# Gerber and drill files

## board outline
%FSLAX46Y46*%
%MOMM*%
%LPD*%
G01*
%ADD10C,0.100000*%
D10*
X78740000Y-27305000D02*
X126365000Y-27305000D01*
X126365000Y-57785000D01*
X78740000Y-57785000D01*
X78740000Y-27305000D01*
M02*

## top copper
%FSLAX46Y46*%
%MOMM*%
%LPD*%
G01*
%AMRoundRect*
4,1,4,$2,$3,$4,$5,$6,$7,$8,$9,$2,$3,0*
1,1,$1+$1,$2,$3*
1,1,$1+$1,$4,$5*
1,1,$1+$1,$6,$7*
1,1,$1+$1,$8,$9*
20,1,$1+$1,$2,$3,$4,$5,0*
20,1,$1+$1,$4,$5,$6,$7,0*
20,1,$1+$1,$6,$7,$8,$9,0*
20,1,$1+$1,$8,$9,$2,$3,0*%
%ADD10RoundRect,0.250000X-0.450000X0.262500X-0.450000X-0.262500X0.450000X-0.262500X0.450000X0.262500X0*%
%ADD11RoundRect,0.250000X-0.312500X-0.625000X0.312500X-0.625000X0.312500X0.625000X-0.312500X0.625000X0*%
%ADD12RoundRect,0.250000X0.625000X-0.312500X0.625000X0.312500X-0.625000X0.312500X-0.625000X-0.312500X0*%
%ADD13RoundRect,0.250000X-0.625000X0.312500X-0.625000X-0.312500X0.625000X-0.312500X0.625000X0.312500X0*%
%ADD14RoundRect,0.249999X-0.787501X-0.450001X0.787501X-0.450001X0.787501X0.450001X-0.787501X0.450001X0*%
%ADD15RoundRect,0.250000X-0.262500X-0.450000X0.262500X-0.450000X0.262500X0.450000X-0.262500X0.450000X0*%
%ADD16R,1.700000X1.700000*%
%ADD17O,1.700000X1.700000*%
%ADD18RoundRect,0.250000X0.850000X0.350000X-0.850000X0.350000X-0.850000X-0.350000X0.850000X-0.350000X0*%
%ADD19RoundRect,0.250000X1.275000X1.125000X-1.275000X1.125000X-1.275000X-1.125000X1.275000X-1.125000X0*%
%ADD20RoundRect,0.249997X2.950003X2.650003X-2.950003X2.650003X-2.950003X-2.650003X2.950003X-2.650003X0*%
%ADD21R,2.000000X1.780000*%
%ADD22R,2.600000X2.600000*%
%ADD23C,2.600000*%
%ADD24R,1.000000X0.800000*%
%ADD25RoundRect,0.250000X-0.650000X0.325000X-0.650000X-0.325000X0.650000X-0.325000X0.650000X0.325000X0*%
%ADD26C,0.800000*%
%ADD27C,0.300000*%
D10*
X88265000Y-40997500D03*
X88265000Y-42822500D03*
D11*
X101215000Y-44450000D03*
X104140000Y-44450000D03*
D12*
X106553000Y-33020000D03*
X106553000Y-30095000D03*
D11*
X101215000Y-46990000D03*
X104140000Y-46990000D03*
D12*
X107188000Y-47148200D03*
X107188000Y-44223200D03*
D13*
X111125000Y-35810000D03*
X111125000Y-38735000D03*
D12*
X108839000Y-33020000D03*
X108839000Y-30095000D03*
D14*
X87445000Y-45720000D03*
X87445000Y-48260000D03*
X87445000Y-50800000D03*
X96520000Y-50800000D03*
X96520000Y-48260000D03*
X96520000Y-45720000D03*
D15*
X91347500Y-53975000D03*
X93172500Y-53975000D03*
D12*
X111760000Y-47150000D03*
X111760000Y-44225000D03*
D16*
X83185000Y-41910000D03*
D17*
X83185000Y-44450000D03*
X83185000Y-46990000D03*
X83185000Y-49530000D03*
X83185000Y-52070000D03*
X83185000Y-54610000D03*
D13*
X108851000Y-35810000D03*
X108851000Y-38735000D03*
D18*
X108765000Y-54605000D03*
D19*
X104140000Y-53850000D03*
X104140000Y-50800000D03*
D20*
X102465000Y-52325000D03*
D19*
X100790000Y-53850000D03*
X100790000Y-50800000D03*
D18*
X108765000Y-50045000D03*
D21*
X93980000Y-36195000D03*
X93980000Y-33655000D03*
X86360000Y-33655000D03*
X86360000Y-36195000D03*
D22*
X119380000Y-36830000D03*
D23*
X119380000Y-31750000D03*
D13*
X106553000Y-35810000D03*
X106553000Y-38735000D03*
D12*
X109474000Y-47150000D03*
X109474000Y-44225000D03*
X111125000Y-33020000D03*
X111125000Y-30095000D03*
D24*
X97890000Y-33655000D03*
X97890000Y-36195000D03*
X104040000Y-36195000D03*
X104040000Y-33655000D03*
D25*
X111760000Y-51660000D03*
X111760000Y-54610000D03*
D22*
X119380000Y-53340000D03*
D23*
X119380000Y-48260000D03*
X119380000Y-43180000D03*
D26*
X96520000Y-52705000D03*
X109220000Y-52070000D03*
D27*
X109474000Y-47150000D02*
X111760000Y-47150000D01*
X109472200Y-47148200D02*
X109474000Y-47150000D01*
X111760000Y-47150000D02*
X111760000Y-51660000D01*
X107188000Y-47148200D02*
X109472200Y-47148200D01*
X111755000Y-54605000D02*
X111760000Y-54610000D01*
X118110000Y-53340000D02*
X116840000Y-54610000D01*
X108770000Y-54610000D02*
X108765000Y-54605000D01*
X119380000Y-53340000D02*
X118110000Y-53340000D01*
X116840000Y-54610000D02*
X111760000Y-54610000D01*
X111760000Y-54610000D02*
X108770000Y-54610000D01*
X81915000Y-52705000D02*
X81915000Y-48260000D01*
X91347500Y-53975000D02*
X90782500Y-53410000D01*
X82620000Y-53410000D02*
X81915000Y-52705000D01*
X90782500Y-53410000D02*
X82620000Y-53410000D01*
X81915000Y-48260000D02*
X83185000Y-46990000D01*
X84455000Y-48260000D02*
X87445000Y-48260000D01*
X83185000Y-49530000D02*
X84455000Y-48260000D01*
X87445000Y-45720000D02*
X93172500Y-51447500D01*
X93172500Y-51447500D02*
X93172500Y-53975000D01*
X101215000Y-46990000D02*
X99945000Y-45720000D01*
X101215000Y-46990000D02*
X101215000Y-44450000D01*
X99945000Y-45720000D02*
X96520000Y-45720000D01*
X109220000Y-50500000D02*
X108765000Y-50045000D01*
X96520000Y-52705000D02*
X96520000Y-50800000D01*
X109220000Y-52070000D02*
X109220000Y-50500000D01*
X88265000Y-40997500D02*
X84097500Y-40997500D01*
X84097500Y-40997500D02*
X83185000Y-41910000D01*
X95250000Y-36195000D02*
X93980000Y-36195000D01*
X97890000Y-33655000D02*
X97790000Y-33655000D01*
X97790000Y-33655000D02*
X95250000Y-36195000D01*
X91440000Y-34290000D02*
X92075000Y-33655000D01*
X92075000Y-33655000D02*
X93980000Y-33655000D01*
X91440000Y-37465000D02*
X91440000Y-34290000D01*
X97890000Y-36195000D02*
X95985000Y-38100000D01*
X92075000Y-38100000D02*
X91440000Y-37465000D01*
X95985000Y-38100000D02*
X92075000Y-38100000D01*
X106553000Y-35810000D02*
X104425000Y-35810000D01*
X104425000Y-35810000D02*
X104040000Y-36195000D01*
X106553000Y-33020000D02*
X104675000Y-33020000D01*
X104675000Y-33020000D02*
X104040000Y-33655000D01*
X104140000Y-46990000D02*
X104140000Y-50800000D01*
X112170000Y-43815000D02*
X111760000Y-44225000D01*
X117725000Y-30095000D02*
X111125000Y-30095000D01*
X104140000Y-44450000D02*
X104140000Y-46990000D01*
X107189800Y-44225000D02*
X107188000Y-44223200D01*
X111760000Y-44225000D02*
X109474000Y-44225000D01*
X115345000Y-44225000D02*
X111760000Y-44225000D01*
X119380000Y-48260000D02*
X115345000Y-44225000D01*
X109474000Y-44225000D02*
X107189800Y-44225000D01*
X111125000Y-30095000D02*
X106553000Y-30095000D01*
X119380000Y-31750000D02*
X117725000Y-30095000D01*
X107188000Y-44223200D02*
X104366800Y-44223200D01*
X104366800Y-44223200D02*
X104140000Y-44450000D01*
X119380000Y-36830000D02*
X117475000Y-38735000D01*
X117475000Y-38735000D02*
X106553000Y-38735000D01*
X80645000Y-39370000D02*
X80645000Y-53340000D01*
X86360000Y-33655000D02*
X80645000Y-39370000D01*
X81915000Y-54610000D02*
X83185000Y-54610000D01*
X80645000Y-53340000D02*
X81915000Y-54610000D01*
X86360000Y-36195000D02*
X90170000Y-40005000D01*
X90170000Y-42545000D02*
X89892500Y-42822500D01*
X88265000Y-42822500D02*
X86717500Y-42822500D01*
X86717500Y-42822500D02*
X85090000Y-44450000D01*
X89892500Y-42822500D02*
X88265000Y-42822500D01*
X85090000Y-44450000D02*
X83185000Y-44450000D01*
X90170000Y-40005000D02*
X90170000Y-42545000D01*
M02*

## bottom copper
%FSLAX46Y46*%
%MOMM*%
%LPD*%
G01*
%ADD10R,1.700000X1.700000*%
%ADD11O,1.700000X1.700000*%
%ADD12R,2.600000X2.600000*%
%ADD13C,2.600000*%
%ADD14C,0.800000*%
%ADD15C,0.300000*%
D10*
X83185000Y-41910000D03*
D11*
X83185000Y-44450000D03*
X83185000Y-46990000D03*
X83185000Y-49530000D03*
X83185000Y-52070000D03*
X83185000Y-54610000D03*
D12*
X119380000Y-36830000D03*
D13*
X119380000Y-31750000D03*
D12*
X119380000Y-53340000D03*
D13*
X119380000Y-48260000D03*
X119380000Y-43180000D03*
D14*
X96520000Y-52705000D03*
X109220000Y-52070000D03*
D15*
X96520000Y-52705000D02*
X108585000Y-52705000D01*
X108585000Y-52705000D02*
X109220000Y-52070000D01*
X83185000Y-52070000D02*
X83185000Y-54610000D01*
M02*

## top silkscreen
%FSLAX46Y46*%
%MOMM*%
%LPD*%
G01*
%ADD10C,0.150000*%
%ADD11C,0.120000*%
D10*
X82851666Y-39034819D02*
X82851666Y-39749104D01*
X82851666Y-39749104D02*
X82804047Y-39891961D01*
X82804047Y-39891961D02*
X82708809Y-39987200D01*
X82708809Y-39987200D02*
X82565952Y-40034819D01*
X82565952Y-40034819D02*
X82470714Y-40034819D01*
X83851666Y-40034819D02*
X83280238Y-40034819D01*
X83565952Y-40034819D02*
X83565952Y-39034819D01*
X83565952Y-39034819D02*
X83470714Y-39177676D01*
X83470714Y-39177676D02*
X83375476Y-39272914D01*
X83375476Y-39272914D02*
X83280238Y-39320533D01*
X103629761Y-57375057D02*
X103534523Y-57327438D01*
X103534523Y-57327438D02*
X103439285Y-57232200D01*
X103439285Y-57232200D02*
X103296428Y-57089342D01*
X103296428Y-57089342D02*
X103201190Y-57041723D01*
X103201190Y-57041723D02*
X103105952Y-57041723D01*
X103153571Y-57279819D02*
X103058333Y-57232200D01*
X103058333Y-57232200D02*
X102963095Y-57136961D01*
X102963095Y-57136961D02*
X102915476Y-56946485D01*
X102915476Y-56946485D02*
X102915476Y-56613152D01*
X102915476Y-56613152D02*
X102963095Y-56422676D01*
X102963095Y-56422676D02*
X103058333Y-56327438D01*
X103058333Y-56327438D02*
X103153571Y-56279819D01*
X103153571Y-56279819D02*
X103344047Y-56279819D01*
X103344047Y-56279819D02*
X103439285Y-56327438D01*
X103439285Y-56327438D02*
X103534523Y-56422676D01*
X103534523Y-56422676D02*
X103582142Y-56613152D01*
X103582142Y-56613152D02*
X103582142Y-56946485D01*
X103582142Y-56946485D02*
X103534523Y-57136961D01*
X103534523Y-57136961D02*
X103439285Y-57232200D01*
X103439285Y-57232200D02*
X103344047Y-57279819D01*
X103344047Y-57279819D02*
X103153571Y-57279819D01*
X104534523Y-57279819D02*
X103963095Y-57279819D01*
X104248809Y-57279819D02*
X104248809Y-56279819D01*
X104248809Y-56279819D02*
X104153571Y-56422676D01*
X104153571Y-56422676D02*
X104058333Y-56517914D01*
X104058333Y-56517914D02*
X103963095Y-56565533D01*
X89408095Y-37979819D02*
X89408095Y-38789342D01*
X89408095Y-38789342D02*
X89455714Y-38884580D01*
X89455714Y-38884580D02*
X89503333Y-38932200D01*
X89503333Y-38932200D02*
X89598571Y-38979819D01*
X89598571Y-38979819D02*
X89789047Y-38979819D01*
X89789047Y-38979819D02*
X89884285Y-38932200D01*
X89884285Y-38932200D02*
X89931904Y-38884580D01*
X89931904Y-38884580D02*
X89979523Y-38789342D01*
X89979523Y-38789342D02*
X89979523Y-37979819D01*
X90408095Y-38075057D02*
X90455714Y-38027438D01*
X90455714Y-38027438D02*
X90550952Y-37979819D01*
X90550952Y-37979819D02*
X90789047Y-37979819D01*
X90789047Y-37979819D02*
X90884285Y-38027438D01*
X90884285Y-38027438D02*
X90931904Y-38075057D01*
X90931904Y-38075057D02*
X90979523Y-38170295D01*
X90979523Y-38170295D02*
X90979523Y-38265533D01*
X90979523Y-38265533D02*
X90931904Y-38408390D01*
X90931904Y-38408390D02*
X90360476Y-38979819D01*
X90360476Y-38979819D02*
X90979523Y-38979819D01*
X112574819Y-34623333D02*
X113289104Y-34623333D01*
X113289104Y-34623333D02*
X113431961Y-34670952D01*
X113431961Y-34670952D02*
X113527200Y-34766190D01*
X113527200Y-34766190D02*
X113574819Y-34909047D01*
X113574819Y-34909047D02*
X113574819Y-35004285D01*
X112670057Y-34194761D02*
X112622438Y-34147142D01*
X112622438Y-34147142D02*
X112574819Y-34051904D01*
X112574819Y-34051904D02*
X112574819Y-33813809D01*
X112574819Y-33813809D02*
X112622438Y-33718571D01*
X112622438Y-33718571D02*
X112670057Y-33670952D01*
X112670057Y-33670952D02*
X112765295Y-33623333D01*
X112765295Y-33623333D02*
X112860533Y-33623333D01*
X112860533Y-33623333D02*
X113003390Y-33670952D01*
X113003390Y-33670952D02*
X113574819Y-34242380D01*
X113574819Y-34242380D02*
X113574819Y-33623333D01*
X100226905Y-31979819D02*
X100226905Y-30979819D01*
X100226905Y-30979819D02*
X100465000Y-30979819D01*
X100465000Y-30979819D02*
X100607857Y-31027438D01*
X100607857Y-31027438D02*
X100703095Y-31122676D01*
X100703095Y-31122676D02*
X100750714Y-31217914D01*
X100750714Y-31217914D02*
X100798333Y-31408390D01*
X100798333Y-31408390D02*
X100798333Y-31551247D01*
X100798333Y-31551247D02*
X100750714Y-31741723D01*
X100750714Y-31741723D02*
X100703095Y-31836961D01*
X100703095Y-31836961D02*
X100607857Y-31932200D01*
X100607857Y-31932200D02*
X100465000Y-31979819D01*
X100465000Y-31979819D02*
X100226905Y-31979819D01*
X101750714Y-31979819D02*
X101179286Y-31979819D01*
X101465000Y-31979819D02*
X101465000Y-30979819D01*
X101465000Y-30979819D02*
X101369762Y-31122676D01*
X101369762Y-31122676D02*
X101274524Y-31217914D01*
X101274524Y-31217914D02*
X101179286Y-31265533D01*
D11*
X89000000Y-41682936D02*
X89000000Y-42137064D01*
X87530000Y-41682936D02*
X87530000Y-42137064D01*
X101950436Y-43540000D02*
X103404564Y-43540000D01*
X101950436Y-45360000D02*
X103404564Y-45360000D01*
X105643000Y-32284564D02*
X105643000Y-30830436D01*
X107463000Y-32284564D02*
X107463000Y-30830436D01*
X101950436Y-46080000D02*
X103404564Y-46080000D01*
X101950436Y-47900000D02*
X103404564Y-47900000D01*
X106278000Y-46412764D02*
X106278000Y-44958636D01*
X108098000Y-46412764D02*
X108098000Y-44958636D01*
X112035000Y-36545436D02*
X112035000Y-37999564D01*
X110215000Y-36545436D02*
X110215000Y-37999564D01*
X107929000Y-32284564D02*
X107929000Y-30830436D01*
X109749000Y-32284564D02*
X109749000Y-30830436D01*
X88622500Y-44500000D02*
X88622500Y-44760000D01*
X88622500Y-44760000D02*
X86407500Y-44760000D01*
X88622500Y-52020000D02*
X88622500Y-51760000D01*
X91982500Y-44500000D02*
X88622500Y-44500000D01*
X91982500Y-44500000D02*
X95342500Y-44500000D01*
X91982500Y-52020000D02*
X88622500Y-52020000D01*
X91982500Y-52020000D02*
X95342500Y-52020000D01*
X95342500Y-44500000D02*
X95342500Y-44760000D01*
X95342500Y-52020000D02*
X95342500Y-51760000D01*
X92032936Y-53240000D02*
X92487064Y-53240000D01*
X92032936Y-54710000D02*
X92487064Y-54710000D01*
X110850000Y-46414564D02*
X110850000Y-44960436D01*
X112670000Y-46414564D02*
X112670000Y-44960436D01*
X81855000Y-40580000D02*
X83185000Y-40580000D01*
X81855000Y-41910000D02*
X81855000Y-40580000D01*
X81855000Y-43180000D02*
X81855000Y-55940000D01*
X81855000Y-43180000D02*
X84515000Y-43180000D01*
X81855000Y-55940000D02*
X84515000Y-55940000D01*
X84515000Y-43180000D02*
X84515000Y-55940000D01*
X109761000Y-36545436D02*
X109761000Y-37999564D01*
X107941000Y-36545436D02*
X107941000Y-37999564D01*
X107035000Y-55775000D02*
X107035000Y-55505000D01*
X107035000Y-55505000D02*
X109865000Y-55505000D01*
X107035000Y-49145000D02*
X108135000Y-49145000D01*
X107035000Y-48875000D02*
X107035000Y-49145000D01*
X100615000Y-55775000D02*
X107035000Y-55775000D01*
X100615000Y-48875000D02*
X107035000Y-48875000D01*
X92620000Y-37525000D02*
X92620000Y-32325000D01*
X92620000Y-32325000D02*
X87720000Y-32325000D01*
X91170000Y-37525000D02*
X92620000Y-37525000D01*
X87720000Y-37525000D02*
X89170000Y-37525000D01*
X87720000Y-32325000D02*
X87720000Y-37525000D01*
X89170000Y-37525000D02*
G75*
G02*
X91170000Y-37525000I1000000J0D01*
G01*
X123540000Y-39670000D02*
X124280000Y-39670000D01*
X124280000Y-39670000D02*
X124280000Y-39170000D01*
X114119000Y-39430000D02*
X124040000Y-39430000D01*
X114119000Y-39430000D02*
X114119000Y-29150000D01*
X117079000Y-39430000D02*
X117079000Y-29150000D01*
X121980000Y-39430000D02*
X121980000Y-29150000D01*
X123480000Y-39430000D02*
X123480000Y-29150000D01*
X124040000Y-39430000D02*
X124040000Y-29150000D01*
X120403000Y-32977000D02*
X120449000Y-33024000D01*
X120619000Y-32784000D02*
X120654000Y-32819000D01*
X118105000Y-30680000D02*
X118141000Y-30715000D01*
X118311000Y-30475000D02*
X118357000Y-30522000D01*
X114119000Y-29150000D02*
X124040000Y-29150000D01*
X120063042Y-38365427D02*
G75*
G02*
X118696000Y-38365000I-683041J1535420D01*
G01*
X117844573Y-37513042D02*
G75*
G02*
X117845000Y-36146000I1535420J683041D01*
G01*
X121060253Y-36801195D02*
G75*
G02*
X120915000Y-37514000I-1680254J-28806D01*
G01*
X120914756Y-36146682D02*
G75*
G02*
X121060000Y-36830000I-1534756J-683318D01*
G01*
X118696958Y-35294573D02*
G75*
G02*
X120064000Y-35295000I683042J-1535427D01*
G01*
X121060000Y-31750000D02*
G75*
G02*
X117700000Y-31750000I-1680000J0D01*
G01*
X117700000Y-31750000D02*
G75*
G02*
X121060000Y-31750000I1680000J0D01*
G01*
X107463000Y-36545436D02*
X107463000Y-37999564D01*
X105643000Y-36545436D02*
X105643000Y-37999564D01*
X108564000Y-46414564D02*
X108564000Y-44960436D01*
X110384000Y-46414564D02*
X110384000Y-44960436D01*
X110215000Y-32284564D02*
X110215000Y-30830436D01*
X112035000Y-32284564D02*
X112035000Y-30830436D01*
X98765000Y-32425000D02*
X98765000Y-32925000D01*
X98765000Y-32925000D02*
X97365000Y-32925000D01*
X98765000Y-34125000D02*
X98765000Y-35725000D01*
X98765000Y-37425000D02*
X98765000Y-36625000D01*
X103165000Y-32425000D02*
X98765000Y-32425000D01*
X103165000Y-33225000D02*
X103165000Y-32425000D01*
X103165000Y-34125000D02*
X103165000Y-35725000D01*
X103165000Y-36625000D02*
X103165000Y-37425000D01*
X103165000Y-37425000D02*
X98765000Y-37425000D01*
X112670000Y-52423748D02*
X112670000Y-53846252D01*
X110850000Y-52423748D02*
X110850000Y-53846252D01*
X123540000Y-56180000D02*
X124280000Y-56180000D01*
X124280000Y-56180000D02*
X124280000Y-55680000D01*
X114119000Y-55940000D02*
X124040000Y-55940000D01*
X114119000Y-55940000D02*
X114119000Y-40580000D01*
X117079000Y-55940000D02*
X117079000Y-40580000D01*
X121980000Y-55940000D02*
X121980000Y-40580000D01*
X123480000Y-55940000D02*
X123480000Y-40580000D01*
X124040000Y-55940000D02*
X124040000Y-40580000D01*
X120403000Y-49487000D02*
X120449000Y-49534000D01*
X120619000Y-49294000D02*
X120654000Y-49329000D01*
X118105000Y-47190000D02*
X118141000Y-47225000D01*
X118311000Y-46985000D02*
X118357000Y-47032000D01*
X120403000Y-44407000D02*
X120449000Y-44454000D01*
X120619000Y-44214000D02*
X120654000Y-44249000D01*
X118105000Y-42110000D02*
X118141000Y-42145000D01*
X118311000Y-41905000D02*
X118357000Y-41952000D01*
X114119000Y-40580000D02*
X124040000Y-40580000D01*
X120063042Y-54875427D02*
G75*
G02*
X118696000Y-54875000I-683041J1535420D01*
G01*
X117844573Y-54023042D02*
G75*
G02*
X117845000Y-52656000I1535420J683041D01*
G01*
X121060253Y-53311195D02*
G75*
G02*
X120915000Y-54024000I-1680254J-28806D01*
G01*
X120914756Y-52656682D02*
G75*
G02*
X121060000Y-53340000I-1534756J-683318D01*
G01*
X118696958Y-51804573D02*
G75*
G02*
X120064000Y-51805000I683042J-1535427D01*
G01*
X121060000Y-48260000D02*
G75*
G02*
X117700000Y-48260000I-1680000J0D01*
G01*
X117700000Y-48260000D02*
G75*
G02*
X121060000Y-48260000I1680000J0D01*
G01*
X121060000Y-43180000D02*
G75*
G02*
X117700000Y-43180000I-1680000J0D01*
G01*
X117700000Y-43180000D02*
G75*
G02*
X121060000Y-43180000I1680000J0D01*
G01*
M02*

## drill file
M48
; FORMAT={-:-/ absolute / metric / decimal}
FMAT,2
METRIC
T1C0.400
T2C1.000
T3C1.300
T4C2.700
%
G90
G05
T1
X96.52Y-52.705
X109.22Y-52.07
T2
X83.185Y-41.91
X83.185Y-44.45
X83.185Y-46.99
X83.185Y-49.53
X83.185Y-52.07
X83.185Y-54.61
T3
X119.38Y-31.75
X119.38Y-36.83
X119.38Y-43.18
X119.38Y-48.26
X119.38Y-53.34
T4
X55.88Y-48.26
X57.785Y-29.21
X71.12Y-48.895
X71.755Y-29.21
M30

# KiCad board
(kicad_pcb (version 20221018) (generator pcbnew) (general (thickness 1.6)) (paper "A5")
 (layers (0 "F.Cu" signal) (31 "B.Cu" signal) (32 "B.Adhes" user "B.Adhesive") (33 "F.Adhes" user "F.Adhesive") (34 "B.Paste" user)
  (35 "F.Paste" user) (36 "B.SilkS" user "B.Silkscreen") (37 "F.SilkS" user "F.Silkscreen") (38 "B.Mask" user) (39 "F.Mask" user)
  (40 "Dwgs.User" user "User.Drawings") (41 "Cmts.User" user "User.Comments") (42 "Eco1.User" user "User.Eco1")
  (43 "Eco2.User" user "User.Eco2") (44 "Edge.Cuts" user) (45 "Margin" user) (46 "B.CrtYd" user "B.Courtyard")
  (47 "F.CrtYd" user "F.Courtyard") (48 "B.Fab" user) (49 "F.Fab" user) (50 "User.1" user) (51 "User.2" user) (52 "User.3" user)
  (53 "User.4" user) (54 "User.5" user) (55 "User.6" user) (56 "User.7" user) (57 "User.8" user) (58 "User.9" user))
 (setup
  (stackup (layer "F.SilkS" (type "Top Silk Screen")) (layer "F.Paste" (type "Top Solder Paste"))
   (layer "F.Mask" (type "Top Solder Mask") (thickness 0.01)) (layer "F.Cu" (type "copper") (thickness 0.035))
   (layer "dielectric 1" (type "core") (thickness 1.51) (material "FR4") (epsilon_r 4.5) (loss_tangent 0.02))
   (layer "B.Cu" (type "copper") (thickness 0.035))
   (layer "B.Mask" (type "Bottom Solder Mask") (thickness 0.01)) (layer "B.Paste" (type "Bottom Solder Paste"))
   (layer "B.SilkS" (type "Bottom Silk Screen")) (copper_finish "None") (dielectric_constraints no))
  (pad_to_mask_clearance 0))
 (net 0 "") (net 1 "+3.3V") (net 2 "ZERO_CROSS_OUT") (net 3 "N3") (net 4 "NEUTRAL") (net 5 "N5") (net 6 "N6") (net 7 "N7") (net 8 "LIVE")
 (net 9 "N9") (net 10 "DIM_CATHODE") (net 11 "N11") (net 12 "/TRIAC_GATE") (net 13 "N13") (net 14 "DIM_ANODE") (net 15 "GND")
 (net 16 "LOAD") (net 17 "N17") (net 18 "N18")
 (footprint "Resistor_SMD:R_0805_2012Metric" (layer "F.Cu") (at 88.265 41.91 -90)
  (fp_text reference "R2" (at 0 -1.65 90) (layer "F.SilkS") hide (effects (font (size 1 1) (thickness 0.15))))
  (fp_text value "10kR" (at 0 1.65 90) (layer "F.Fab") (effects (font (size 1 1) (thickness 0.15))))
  (fp_line (start -0.227064 -0.735) (end 0.227064 -0.735) (stroke (width 0.12) (type solid)) (layer "F.SilkS"))
  (fp_line (start -0.227064 0.735) (end 0.227064 0.735) (stroke (width 0.12) (type solid)) (layer "F.SilkS"))
  (pad "1" smd roundrect (at -0.9125 0 270) (size 1.025 1.4) (layers "F.Cu" "F.Paste" "F.Mask") (roundrect_rratio 0.243902) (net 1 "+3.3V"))
  (pad "2" smd roundrect (at 0.9125 0 270) (size 1.025 1.4) (layers "F.Cu" "F.Paste" "F.Mask") (roundrect_rratio 0.243902)
   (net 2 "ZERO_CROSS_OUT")))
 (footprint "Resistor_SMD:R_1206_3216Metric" (layer "F.Cu") (at 102.6775 44.45)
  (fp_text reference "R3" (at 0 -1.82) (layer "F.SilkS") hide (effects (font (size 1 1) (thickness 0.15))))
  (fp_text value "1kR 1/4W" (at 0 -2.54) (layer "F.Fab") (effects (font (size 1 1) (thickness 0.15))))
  (fp_line (start -0.727064 -0.91) (end 0.727064 -0.91) (stroke (width 0.12) (type solid)) (layer "F.SilkS"))
  (fp_line (start -0.727064 0.91) (end 0.727064 0.91) (stroke (width 0.12) (type solid)) (layer "F.SilkS"))
  (pad "1" smd roundrect (at -1.4625 0) (size 1.125 1.75) (layers "F.Cu" "F.Paste" "F.Mask") (roundrect_rratio 0.2222222222) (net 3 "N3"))
  (pad "2" smd roundrect (at 1.4625 0) (size 1.125 1.75) (layers "F.Cu" "F.Paste" "F.Mask") (roundrect_rratio 0.2222222222)
   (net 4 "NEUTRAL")))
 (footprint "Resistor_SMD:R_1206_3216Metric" (layer "F.Cu") (at 106.553 31.5575 90)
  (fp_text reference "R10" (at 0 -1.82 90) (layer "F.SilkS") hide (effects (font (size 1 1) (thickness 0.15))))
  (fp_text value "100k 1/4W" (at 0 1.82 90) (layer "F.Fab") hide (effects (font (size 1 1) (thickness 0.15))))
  (fp_line (start -0.727064 -0.91) (end 0.727064 -0.91) (stroke (width 0.12) (type solid)) (layer "F.SilkS"))
  (fp_line (start -0.727064 0.91) (end 0.727064 0.91) (stroke (width 0.12) (type solid)) (layer "F.SilkS"))
  (pad "1" smd roundrect (at -1.4625 0 90) (size 1.125 1.75) (layers "F.Cu" "F.Paste" "F.Mask") (roundrect_rratio 0.222222) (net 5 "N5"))
  (pad "2" smd roundrect (at 1.4625 0 90) (size 1.125 1.75) (layers "F.Cu" "F.Paste" "F.Mask") (roundrect_rratio 0.222222) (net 4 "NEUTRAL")))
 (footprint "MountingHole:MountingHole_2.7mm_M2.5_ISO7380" (layer "F.Cu") (at 71.755 29.21)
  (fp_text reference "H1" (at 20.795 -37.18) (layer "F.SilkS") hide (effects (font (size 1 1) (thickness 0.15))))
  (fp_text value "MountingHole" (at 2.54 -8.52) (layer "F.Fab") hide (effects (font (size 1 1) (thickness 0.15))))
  (pad "" np_thru_hole circle (at 0 0) (size 2.7 2.7) (drill 2.7) (layers "*.Cu" "*.Mask")))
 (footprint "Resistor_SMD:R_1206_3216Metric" (layer "F.Cu") (at 102.6775 46.99)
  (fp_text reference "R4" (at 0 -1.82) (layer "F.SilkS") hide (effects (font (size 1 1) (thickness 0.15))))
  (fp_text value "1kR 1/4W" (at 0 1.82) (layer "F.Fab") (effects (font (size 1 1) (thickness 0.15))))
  (fp_line (start -0.727064 -0.91) (end 0.727064 -0.91) (stroke (width 0.12) (type solid)) (layer "F.SilkS"))
  (fp_line (start -0.727064 0.91) (end 0.727064 0.91) (stroke (width 0.12) (type solid)) (layer "F.SilkS"))
  (pad "1" smd roundrect (at -1.4625 0) (size 1.125 1.75) (layers "F.Cu" "F.Paste" "F.Mask") (roundrect_rratio 0.2222222222) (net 3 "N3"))
  (pad "2" smd roundrect (at 1.4625 0) (size 1.125 1.75) (layers "F.Cu" "F.Paste" "F.Mask") (roundrect_rratio 0.2222222222)
   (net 4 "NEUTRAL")))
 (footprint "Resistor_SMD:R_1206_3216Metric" (layer "F.Cu") (at 107.188 45.6857 90)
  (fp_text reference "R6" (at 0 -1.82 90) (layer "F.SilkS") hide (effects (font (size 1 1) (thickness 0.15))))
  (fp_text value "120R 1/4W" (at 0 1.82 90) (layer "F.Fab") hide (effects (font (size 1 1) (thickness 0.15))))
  (fp_line (start -0.727064 -0.91) (end 0.727064 -0.91) (stroke (width 0.12) (type solid)) (layer "F.SilkS"))
  (fp_line (start -0.727064 0.91) (end 0.727064 0.91) (stroke (width 0.12) (type solid)) (layer "F.SilkS"))
  (pad "1" smd roundrect (at -1.4625 0 90) (size 1.125 1.75) (layers "F.Cu" "F.Paste" "F.Mask") (roundrect_rratio 0.222222) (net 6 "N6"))
  (pad "2" smd roundrect (at 1.4625 0 90) (size 1.125 1.75) (layers "F.Cu" "F.Paste" "F.Mask") (roundrect_rratio 0.222222) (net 4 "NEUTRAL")))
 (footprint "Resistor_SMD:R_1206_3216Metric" (layer "F.Cu") (at 111.125 37.2725 -90)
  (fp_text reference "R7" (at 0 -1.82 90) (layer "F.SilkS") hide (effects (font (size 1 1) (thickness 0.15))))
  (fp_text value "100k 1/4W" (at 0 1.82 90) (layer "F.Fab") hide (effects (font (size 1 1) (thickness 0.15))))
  (fp_line (start -0.727064 -0.91) (end 0.727064 -0.91) (stroke (width 0.12) (type solid)) (layer "F.SilkS"))
  (fp_line (start -0.727064 0.91) (end 0.727064 0.91) (stroke (width 0.12) (type solid)) (layer "F.SilkS"))
  (pad "1" smd roundrect (at -1.4625 0 270) (size 1.125 1.75) (layers "F.Cu" "F.Paste" "F.Mask") (roundrect_rratio 0.222222) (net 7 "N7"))
  (pad "2" smd roundrect (at 1.4625 0 270) (size 1.125 1.75) (layers "F.Cu" "F.Paste" "F.Mask") (roundrect_rratio 0.222222) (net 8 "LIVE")))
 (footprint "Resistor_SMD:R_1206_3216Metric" (layer "F.Cu") (at 108.839 31.5575 90)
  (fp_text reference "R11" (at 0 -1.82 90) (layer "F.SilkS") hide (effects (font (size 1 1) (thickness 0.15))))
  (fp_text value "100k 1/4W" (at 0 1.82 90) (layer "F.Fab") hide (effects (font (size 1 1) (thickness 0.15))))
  (fp_line (start -0.727064 -0.91) (end 0.727064 -0.91) (stroke (width 0.12) (type solid)) (layer "F.SilkS"))
  (fp_line (start -0.727064 0.91) (end 0.727064 0.91) (stroke (width 0.12) (type solid)) (layer "F.SilkS"))
  (pad "1" smd roundrect (at -1.4625 0 90) (size 1.125 1.75) (layers "F.Cu" "F.Paste" "F.Mask") (roundrect_rratio 0.222222) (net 5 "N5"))
  (pad "2" smd roundrect (at 1.4625 0 90) (size 1.125 1.75) (layers "F.Cu" "F.Paste" "F.Mask") (roundrect_rratio 0.222222) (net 4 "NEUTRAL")))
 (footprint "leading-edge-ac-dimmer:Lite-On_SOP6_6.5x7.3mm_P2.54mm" (layer "F.Cu") (at 91.9825 48.26)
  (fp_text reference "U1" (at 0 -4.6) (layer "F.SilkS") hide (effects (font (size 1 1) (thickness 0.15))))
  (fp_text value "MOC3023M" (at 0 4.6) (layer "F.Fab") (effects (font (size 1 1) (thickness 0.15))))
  (fp_line (start -3.36 -3.76) (end -3.36 -3.5) (stroke (width 0.12) (type solid)) (layer "F.SilkS"))
  (fp_line (start -3.36 -3.5) (end -5.575 -3.5) (stroke (width 0.12) (type solid)) (layer "F.SilkS"))
  (fp_line (start -3.36 3.76) (end -3.36 3.5) (stroke (width 0.12) (type solid)) (layer "F.SilkS"))
  (fp_line (start 0 -3.76) (end -3.36 -3.76) (stroke (width 0.12) (type solid)) (layer "F.SilkS"))
  (fp_line (start 0 -3.76) (end 3.36 -3.76) (stroke (width 0.12) (type solid)) (layer "F.SilkS"))
  (fp_line (start 0 3.76) (end -3.36 3.76) (stroke (width 0.12) (type solid)) (layer "F.SilkS"))
  (fp_line (start 0 3.76) (end 3.36 3.76) (stroke (width 0.12) (type solid)) (layer "F.SilkS"))
  (fp_line (start 3.36 -3.76) (end 3.36 -3.5) (stroke (width 0.12) (type solid)) (layer "F.SilkS"))
  (fp_line (start 3.36 3.76) (end 3.36 3.5) (stroke (width 0.12) (type solid)) (layer "F.SilkS"))
  (pad "1" smd roundrect (at -4.5375 -2.54) (size 2.075 1.4) (layers "F.Cu" "F.Paste" "F.Mask") (roundrect_rratio 0.178571) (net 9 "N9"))
  (pad "2" smd roundrect (at -4.5375 0) (size 2.075 1.4) (layers "F.Cu" "F.Paste" "F.Mask") (roundrect_rratio 0.178571)
   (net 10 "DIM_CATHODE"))
  (pad "3" smd roundrect (at -4.5375 2.54) (size 2.075 1.4) (layers "F.Cu" "F.Paste" "F.Mask") (roundrect_rratio 0.178571) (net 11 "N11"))
  (pad "4" smd roundrect (at 4.5375 2.54) (size 2.075 1.4) (layers "F.Cu" "F.Paste" "F.Mask") (roundrect_rratio 0.178571)
   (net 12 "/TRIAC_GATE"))
  (pad "5" smd roundrect (at 4.5375 0) (size 2.075 1.4) (layers "F.Cu" "F.Paste" "F.Mask") (roundrect_rratio 0.178571) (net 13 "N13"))
  (pad "6" smd roundrect (at 4.5375 -2.54) (size 2.075 1.4) (layers "F.Cu" "F.Paste" "F.Mask") (roundrect_rratio 0.178571) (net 3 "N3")))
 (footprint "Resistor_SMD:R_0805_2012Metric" (layer "F.Cu") (at 92.26 53.975)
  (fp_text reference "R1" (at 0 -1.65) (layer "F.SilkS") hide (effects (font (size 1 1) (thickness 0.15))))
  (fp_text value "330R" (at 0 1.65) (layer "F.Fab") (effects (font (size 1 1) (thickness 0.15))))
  (fp_line (start -0.227064 -0.735) (end 0.227064 -0.735) (stroke (width 0.12) (type solid)) (layer "F.SilkS"))
  (fp_line (start -0.227064 0.735) (end 0.227064 0.735) (stroke (width 0.12) (type solid)) (layer "F.SilkS"))
  (pad "1" smd roundrect (at -0.9125 0) (size 1.025 1.4) (layers "F.Cu" "F.Paste" "F.Mask") (roundrect_rratio 0.243902) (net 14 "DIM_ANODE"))
  (pad "2" smd roundrect (at 0.9125 0) (size 1.025 1.4) (layers "F.Cu" "F.Paste" "F.Mask") (roundrect_rratio 0.243902) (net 9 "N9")))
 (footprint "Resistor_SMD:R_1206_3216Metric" (layer "F.Cu") (at 111.76 45.6875 90)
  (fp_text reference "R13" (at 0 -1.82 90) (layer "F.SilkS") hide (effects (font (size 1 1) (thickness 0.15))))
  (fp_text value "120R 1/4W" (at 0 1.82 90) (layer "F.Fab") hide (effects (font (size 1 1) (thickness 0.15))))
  (fp_line (start -0.727064 -0.91) (end 0.727064 -0.91) (stroke (width 0.12) (type solid)) (layer "F.SilkS"))
  (fp_line (start -0.727064 0.91) (end 0.727064 0.91) (stroke (width 0.12) (type solid)) (layer "F.SilkS"))
  (pad "1" smd roundrect (at -1.4625 0 90) (size 1.125 1.75) (layers "F.Cu" "F.Paste" "F.Mask") (roundrect_rratio 0.222222) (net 6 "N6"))
  (pad "2" smd roundrect (at 1.4625 0 90) (size 1.125 1.75) (layers "F.Cu" "F.Paste" "F.Mask") (roundrect_rratio 0.222222) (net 4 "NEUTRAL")))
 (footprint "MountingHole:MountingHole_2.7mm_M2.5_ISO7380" (layer "F.Cu") (at 55.88 48.26)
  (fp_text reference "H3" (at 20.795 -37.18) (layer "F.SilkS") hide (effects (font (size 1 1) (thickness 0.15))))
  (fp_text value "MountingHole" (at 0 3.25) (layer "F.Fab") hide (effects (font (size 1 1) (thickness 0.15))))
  (pad "" np_thru_hole circle (at 0 0) (size 2.7 2.7) (drill 2.7) (layers "*.Cu" "*.Mask")))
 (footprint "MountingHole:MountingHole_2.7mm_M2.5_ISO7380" (layer "F.Cu") (at 57.785 29.21)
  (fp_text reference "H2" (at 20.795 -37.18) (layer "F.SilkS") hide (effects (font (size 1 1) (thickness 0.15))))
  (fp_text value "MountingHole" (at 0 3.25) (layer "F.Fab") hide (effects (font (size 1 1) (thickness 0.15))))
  (pad "" np_thru_hole circle (at 0 0) (size 2.7 2.7) (drill 2.7) (layers "*.Cu" "*.Mask")))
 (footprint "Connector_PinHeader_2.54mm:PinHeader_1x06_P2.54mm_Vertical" (layer "F.Cu") (at 83.185 41.91)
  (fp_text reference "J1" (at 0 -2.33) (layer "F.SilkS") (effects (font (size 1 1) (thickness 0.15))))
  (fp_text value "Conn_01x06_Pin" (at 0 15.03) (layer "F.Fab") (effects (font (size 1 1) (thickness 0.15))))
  (fp_line (start -1.33 -1.33) (end 0 -1.33) (stroke (width 0.12) (type solid)) (layer "F.SilkS"))
  (fp_line (start -1.33 0) (end -1.33 -1.33) (stroke (width 0.12) (type solid)) (layer "F.SilkS"))
  (fp_line (start -1.33 1.27) (end -1.33 14.03) (stroke (width 0.12) (type solid)) (layer "F.SilkS"))
  (fp_line (start -1.33 1.27) (end 1.33 1.27) (stroke (width 0.12) (type solid)) (layer "F.SilkS"))
  (fp_line (start -1.33 14.03) (end 1.33 14.03) (stroke (width 0.12) (type solid)) (layer "F.SilkS"))
  (fp_line (start 1.33 1.27) (end 1.33 14.03) (stroke (width 0.12) (type solid)) (layer "F.SilkS"))
  (pad "1" thru_hole rect (at 0 0) (size 1.7 1.7) (drill 1) (layers "*.Cu" "*.Mask") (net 1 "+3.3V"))
  (pad "2" thru_hole oval (at 0 2.54) (size 1.7 1.7) (drill 1) (layers "*.Cu" "*.Mask") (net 2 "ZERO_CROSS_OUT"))
  (pad "3" thru_hole oval (at 0 5.08) (size 1.7 1.7) (drill 1) (layers "*.Cu" "*.Mask") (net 14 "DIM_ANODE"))
  (pad "4" thru_hole oval (at 0 7.62) (size 1.7 1.7) (drill 1) (layers "*.Cu" "*.Mask") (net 10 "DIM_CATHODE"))
  (pad "5" thru_hole oval (at 0 10.16) (size 1.7 1.7) (drill 1) (layers "*.Cu" "*.Mask") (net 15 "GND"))
  (pad "6" thru_hole oval (at 0 12.7) (size 1.7 1.7) (drill 1) (layers "*.Cu" "*.Mask") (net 15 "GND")))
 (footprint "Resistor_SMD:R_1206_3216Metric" (layer "F.Cu") (at 108.851 37.2725 -90)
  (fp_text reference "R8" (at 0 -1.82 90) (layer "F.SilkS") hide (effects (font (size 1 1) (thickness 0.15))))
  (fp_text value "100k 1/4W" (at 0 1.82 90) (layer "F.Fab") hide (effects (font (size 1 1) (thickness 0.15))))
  (fp_line (start -0.727064 -0.91) (end 0.727064 -0.91) (stroke (width 0.12) (type solid)) (layer "F.SilkS"))
  (fp_line (start -0.727064 0.91) (end 0.727064 0.91) (stroke (width 0.12) (type solid)) (layer "F.SilkS"))
  (pad "1" smd roundrect (at -1.4625 0 270) (size 1.125 1.75) (layers "F.Cu" "F.Paste" "F.Mask") (roundrect_rratio 0.222222) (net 7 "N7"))
  (pad "2" smd roundrect (at 1.4625 0 270) (size 1.125 1.75) (layers "F.Cu" "F.Paste" "F.Mask") (roundrect_rratio 0.222222) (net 8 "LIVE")))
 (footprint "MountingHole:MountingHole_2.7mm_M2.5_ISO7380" (layer "F.Cu") (at 71.12 48.895)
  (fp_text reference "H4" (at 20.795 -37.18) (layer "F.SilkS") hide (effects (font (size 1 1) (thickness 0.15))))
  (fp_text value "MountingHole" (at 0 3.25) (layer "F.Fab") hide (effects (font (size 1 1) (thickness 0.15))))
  (pad "" np_thru_hole circle (at 0 0) (size 2.7 2.7) (drill 2.7) (layers "*.Cu" "*.Mask")))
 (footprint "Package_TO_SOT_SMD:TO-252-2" (layer "F.Cu") (at 103.725 52.325 180)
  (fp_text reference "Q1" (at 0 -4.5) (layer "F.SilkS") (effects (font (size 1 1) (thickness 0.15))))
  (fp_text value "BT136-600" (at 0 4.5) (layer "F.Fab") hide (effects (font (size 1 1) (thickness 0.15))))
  (fp_line (start -3.31 -3.45) (end -3.31 -3.18) (stroke (width 0.12) (type solid)) (layer "F.SilkS"))
  (fp_line (start -3.31 -3.18) (end -6.14 -3.18) (stroke (width 0.12) (type solid)) (layer "F.SilkS"))
  (fp_line (start -3.31 3.18) (end -4.41 3.18) (stroke (width 0.12) (type solid)) (layer "F.SilkS"))
  (fp_line (start -3.31 3.45) (end -3.31 3.18) (stroke (width 0.12) (type solid)) (layer "F.SilkS"))
  (fp_line (start 3.11 -3.45) (end -3.31 -3.45) (stroke (width 0.12) (type solid)) (layer "F.SilkS"))
  (fp_line (start 3.11 3.45) (end -3.31 3.45) (stroke (width 0.12) (type solid)) (layer "F.SilkS"))
  (pad "1" smd roundrect (at -5.04 -2.28 180) (size 2.2 1.2) (layers "F.Cu" "F.Paste" "F.Mask") (roundrect_rratio 0.208333) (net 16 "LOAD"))
  (pad "2" smd roundrect (at -0.415 -1.525 180) (size 3.05 2.75) (layers "F.Cu" "F.Paste") (roundrect_rratio 0.090909) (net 4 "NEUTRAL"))
  (pad "2" smd roundrect (at -0.415 1.525 180) (size 3.05 2.75) (layers "F.Cu" "F.Paste") (roundrect_rratio 0.090909) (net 4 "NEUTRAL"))
  (pad "2" smd roundrect (at 1.26 0 180) (size 6.4 5.8) (layers "F.Cu" "F.Mask") (roundrect_rratio 0.043103) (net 4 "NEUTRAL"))
  (pad "2" smd roundrect (at 2.935 -1.525 180) (size 3.05 2.75) (layers "F.Cu" "F.Paste") (roundrect_rratio 0.090909) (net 4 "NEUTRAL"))
  (pad "2" smd roundrect (at 2.935 1.525 180) (size 3.05 2.75) (layers "F.Cu" "F.Paste") (roundrect_rratio 0.090909) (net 4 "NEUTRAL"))
  (pad "3" smd roundrect (at -5.04 2.28 180) (size 2.2 1.2) (layers "F.Cu" "F.Paste" "F.Mask") (roundrect_rratio 0.208333)
   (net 12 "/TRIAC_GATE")))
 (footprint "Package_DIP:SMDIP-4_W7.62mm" (layer "F.Cu") (at 90.17 34.925 180)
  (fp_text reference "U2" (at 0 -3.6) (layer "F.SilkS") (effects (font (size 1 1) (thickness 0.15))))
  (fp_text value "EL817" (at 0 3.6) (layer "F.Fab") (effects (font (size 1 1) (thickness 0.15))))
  (fp_line (start -2.45 -2.6) (end -2.45 2.6) (stroke (width 0.12) (type solid)) (layer "F.SilkS"))
  (fp_line (start -2.45 2.6) (end 2.45 2.6) (stroke (width 0.12) (type solid)) (layer "F.SilkS"))
  (fp_line (start -1 -2.6) (end -2.45 -2.6) (stroke (width 0.12) (type solid)) (layer "F.SilkS"))
  (fp_line (start 2.45 -2.6) (end 1 -2.6) (stroke (width 0.12) (type solid)) (layer "F.SilkS"))
  (fp_line (start 2.45 2.6) (end 2.45 -2.6) (stroke (width 0.12) (type solid)) (layer "F.SilkS"))
  (fp_arc (start 1 -2.6) (mid 0 -1.6) (end -1 -2.6) (stroke (width 0.12) (type solid)) (layer "F.SilkS"))
  (pad "1" smd rect (at -3.81 -1.27 180) (size 2 1.78) (layers "F.Cu" "F.Paste" "F.Mask") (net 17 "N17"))
  (pad "2" smd rect (at -3.81 1.27 180) (size 2 1.78) (layers "F.Cu" "F.Paste" "F.Mask") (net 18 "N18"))
  (pad "3" smd rect (at 3.81 1.27 180) (size 2 1.78) (layers "F.Cu" "F.Paste" "F.Mask") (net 15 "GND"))
  (pad "4" smd rect (at 3.81 -1.27 180) (size 2 1.78) (layers "F.Cu" "F.Paste" "F.Mask") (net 2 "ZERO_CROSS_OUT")))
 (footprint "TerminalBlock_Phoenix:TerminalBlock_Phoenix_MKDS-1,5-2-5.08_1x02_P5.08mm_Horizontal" (layer "F.Cu") (at 119.38 36.83 90)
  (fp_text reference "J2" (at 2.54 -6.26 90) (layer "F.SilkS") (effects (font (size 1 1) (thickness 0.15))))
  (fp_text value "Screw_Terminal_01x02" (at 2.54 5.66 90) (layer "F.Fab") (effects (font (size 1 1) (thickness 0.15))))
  (fp_line (start -2.84 4.16) (end -2.84 4.9) (stroke (width 0.12) (type solid)) (layer "F.SilkS"))
  (fp_line (start -2.84 4.9) (end -2.34 4.9) (stroke (width 0.12) (type solid)) (layer "F.SilkS"))
  (fp_line (start -2.6 -5.261) (end -2.6 4.66) (stroke (width 0.12) (type solid)) (layer "F.SilkS"))
  (fp_line (start -2.6 -5.261) (end 7.68 -5.261) (stroke (width 0.12) (type solid)) (layer "F.SilkS"))
  (fp_line (start -2.6 -2.301) (end 7.68 -2.301) (stroke (width 0.12) (type solid)) (layer "F.SilkS"))
  (fp_line (start -2.6 2.6) (end 7.68 2.6) (stroke (width 0.12) (type solid)) (layer "F.SilkS"))
  (fp_line (start -2.6 4.1) (end 7.68 4.1) (stroke (width 0.12) (type solid)) (layer "F.SilkS"))
  (fp_line (start -2.6 4.66) (end 7.68 4.66) (stroke (width 0.12) (type solid)) (layer "F.SilkS"))
  (fp_line (start 3.853 1.023) (end 3.806 1.069) (stroke (width 0.12) (type solid)) (layer "F.SilkS"))
  (fp_line (start 4.046 1.239) (end 4.011 1.274) (stroke (width 0.12) (type solid)) (layer "F.SilkS"))
  (fp_line (start 6.15 -1.275) (end 6.115 -1.239) (stroke (width 0.12) (type solid)) (layer "F.SilkS"))
  (fp_line (start 6.355 -1.069) (end 6.308 -1.023) (stroke (width 0.12) (type solid)) (layer "F.SilkS"))
  (fp_line (start 7.68 -5.261) (end 7.68 4.66) (stroke (width 0.12) (type solid)) (layer "F.SilkS"))
  (fp_arc (start -1.535427 0.683042) (mid -1.680501 -0.000524) (end -1.535 -0.684) (stroke (width 0.12) (type solid)) (layer "F.SilkS"))
  (fp_arc (start -0.683042 -1.535427) (mid 0.000524 -1.680501) (end 0.684 -1.535) (stroke (width 0.12) (type solid)) (layer "F.SilkS"))
  (fp_arc (start 0.028805 1.680253) (mid -0.335551 1.646659) (end -0.684 1.535) (stroke (width 0.12) (type solid)) (layer "F.SilkS"))
  (fp_arc (start 0.683318 1.534756) (mid 0.349292 1.643288) (end 0 1.68) (stroke (width 0.12) (type solid)) (layer "F.SilkS"))
  (fp_arc (start 1.535427 -0.683042) (mid 1.680501 0.000524) (end 1.535 0.684) (stroke (width 0.12) (type solid)) (layer "F.SilkS"))
  (fp_circle (center 5.08 0) (end 6.76 0) (stroke (width 0.12) (type solid)) (fill none) (layer "F.SilkS"))
  (pad "1" thru_hole rect (at 0 0 90) (size 2.6 2.6) (drill 1.3) (layers "*.Cu" "*.Mask") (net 8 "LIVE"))
  (pad "2" thru_hole circle (at 5.08 0 90) (size 2.6 2.6) (drill 1.3) (layers "*.Cu" "*.Mask") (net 4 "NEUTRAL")))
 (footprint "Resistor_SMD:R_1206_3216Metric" (layer "F.Cu") (at 106.553 37.2725 -90)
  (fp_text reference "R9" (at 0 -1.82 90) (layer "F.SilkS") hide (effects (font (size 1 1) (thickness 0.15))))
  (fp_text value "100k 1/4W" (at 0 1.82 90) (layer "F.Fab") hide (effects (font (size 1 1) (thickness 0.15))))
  (fp_line (start -0.727064 -0.91) (end 0.727064 -0.91) (stroke (width 0.12) (type solid)) (layer "F.SilkS"))
  (fp_line (start -0.727064 0.91) (end 0.727064 0.91) (stroke (width 0.12) (type solid)) (layer "F.SilkS"))
  (pad "1" smd roundrect (at -1.4625 0 270) (size 1.125 1.75) (layers "F.Cu" "F.Paste" "F.Mask") (roundrect_rratio 0.222222) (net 7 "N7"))
  (pad "2" smd roundrect (at 1.4625 0 270) (size 1.125 1.75) (layers "F.Cu" "F.Paste" "F.Mask") (roundrect_rratio 0.222222) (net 8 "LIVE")))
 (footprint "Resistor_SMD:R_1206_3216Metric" (layer "F.Cu") (at 109.474 45.6875 90)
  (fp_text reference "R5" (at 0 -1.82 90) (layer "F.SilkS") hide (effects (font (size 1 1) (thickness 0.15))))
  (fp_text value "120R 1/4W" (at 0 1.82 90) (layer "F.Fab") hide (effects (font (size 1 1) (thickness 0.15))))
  (fp_line (start -0.727064 -0.91) (end 0.727064 -0.91) (stroke (width 0.12) (type solid)) (layer "F.SilkS"))
  (fp_line (start -0.727064 0.91) (end 0.727064 0.91) (stroke (width 0.12) (type solid)) (layer "F.SilkS"))
  (pad "1" smd roundrect (at -1.4625 0 90) (size 1.125 1.75) (layers "F.Cu" "F.Paste" "F.Mask") (roundrect_rratio 0.222222) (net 6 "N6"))
  (pad "2" smd roundrect (at 1.4625 0 90) (size 1.125 1.75) (layers "F.Cu" "F.Paste" "F.Mask") (roundrect_rratio 0.222222) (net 4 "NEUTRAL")))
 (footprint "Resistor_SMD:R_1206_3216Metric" (layer "F.Cu") (at 111.125 31.5575 90)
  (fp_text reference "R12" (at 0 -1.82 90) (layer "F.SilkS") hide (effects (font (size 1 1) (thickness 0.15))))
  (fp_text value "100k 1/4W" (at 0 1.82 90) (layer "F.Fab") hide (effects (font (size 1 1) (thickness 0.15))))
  (fp_line (start -0.727064 -0.91) (end 0.727064 -0.91) (stroke (width 0.12) (type solid)) (layer "F.SilkS"))
  (fp_line (start -0.727064 0.91) (end 0.727064 0.91) (stroke (width 0.12) (type solid)) (layer "F.SilkS"))
  (pad "1" smd roundrect (at -1.4625 0 90) (size 1.125 1.75) (layers "F.Cu" "F.Paste" "F.Mask") (roundrect_rratio 0.222222) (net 5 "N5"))
  (pad "2" smd roundrect (at 1.4625 0 90) (size 1.125 1.75) (layers "F.Cu" "F.Paste" "F.Mask") (roundrect_rratio 0.222222) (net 4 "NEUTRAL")))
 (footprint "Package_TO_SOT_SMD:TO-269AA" (layer "F.Cu") (at 100.965 34.925)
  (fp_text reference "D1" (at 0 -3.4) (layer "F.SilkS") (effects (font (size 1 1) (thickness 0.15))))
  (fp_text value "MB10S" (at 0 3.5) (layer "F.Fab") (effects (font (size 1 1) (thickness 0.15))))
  (fp_line (start -2.2 -2.5) (end -2.2 -2) (stroke (width 0.12) (type solid)) (layer "F.SilkS"))
  (fp_line (start -2.2 -2) (end -3.6 -2) (stroke (width 0.12) (type solid)) (layer "F.SilkS"))
  (fp_line (start -2.2 -0.8) (end -2.2 0.8) (stroke (width 0.12) (type solid)) (layer "F.SilkS"))
  (fp_line (start -2.2 2.5) (end -2.2 1.7) (stroke (width 0.12) (type solid)) (layer "F.SilkS"))
  (fp_line (start 2.2 -2.5) (end -2.2 -2.5) (stroke (width 0.12) (type solid)) (layer "F.SilkS"))
  (fp_line (start 2.2 -1.7) (end 2.2 -2.5) (stroke (width 0.12) (type solid)) (layer "F.SilkS"))
  (fp_line (start 2.2 -0.8) (end 2.2 0.8) (stroke (width 0.12) (type solid)) (layer "F.SilkS"))
  (fp_line (start 2.2 1.7) (end 2.2 2.5) (stroke (width 0.12) (type solid)) (layer "F.SilkS"))
  (fp_line (start 2.2 2.5) (end -2.2 2.5) (stroke (width 0.12) (type solid)) (layer "F.SilkS"))
  (pad "1" smd rect (at -3.075 -1.27) (size 1 0.8) (layers "F.Cu" "F.Paste" "F.Mask") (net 17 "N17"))
  (pad "2" smd rect (at -3.075 1.27) (size 1 0.8) (layers "F.Cu" "F.Paste" "F.Mask") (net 18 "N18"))
  (pad "3" smd rect (at 3.075 1.27) (size 1 0.8) (layers "F.Cu" "F.Paste" "F.Mask") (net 7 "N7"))
  (pad "4" smd rect (at 3.075 -1.27) (size 1 0.8) (layers "F.Cu" "F.Paste" "F.Mask") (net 5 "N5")))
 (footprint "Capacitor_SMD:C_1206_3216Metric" (layer "F.Cu") (at 111.76 53.135 -90)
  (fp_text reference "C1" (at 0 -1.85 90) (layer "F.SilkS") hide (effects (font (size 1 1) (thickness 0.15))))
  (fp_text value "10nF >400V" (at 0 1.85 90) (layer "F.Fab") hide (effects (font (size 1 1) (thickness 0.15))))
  (fp_line (start -0.711252 -0.91) (end 0.711252 -0.91) (stroke (width 0.12) (type solid)) (layer "F.SilkS"))
  (fp_line (start -0.711252 0.91) (end 0.711252 0.91) (stroke (width 0.12) (type solid)) (layer "F.SilkS"))
  (pad "1" smd roundrect (at -1.475 0 270) (size 1.15 1.8) (layers "F.Cu" "F.Paste" "F.Mask") (roundrect_rratio 0.217391) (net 6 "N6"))
  (pad "2" smd roundrect (at 1.475 0 270) (size 1.15 1.8) (layers "F.Cu" "F.Paste" "F.Mask") (roundrect_rratio 0.217391) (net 16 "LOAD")))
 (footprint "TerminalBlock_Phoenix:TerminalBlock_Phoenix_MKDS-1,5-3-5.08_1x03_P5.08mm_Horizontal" (layer "F.Cu") (at 119.38 53.34 90)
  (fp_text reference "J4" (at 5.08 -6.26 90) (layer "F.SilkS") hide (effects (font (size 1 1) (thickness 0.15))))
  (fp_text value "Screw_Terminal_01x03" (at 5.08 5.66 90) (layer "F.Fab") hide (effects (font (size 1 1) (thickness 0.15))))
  (fp_line (start -2.84 4.16) (end -2.84 4.9) (stroke (width 0.12) (type solid)) (layer "F.SilkS"))
  (fp_line (start -2.84 4.9) (end -2.34 4.9) (stroke (width 0.12) (type solid)) (layer "F.SilkS"))
  (fp_line (start -2.6 -5.261) (end -2.6 4.66) (stroke (width 0.12) (type solid)) (layer "F.SilkS"))
  (fp_line (start -2.6 -5.261) (end 12.76 -5.261) (stroke (width 0.12) (type solid)) (layer "F.SilkS"))
  (fp_line (start -2.6 -2.301) (end 12.76 -2.301) (stroke (width 0.12) (type solid)) (layer "F.SilkS"))
  (fp_line (start -2.6 2.6) (end 12.76 2.6) (stroke (width 0.12) (type solid)) (layer "F.SilkS"))
  (fp_line (start -2.6 4.1) (end 12.76 4.1) (stroke (width 0.12) (type solid)) (layer "F.SilkS"))
  (fp_line (start -2.6 4.66) (end 12.76 4.66) (stroke (width 0.12) (type solid)) (layer "F.SilkS"))
  (fp_line (start 3.853 1.023) (end 3.806 1.069) (stroke (width 0.12) (type solid)) (layer "F.SilkS"))
  (fp_line (start 4.046 1.239) (end 4.011 1.274) (stroke (width 0.12) (type solid)) (layer "F.SilkS"))
  (fp_line (start 6.15 -1.275) (end 6.115 -1.239) (stroke (width 0.12) (type solid)) (layer "F.SilkS"))
  (fp_line (start 6.355 -1.069) (end 6.308 -1.023) (stroke (width 0.12) (type solid)) (layer "F.SilkS"))
  (fp_line (start 8.933 1.023) (end 8.886 1.069) (stroke (width 0.12) (type solid)) (layer "F.SilkS"))
  (fp_line (start 9.126 1.239) (end 9.091 1.274) (stroke (width 0.12) (type solid)) (layer "F.SilkS"))
  (fp_line (start 11.23 -1.275) (end 11.195 -1.239) (stroke (width 0.12) (type solid)) (layer "F.SilkS"))
  (fp_line (start 11.435 -1.069) (end 11.388 -1.023) (stroke (width 0.12) (type solid)) (layer "F.SilkS"))
  (fp_line (start 12.76 -5.261) (end 12.76 4.66) (stroke (width 0.12) (type solid)) (layer "F.SilkS"))
  (fp_arc (start -1.535427 0.683042) (mid -1.680501 -0.000524) (end -1.535 -0.684) (stroke (width 0.12) (type solid)) (layer "F.SilkS"))
  (fp_arc (start -0.683042 -1.535427) (mid 0.000524 -1.680501) (end 0.684 -1.535) (stroke (width 0.12) (type solid)) (layer "F.SilkS"))
  (fp_arc (start 0.028805 1.680253) (mid -0.335551 1.646659) (end -0.684 1.535) (stroke (width 0.12) (type solid)) (layer "F.SilkS"))
  (fp_arc (start 0.683318 1.534756) (mid 0.349292 1.643288) (end 0 1.68) (stroke (width 0.12) (type solid)) (layer "F.SilkS"))
  (fp_arc (start 1.535427 -0.683042) (mid 1.680501 0.000524) (end 1.535 0.684) (stroke (width 0.12) (type solid)) (layer "F.SilkS"))
  (fp_circle (center 5.08 0) (end 6.76 0) (stroke (width 0.12) (type solid)) (fill none) (layer "F.SilkS"))
  (fp_circle (center 10.16 0) (end 11.84 0) (stroke (width 0.12) (type solid)) (fill none) (layer "F.SilkS"))
  (pad "1" thru_hole rect (at 0 0 90) (size 2.6 2.6) (drill 1.3) (layers "*.Cu" "*.Mask") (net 16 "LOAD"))
  (pad "2" thru_hole circle (at 5.08 0 90) (size 2.6 2.6) (drill 1.3) (layers "*.Cu" "*.Mask") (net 4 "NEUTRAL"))
  (pad "3" thru_hole circle (at 10.16 0 90) (size 2.6 2.6) (drill 1.3) (layers "*.Cu" "*.Mask") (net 8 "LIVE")))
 (gr_rect (start 78.74 27.305) (end 126.365 57.785) (stroke (width 0.1) (type default)) (fill none) (layer "Edge.Cuts"))
 (segment (start 109.474 47.15) (end 111.76 47.15) (width 0.3) (layer "F.Cu") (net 6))
 (segment (start 109.4722 47.1482) (end 109.474 47.15) (width 0.3) (layer "F.Cu") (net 6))
 (segment (start 111.76 47.15) (end 111.76 51.66) (width 0.3) (layer "F.Cu") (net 6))
 (segment (start 107.188 47.1482) (end 109.4722 47.1482) (width 0.3) (layer "F.Cu") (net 6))
 (segment (start 111.755 54.605) (end 111.76 54.61) (width 0.3) (layer "F.Cu") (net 16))
 (segment (start 118.11 53.34) (end 116.84 54.61) (width 0.3) (layer "F.Cu") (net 16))
 (segment (start 108.77 54.61) (end 108.765 54.605) (width 0.3) (layer "F.Cu") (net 16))
 (segment (start 119.38 53.34) (end 118.11 53.34) (width 0.3) (layer "F.Cu") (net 16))
 (segment (start 116.84 54.61) (end 111.76 54.61) (width 0.3) (layer "F.Cu") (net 16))
 (segment (start 111.76 54.61) (end 108.77 54.61) (width 0.3) (layer "F.Cu") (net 16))
 (segment (start 81.915 52.705) (end 81.915 48.26) (width 0.3) (layer "F.Cu") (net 14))
 (segment (start 91.3475 53.975) (end 90.7825 53.41) (width 0.3) (layer "F.Cu") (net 14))
 (segment (start 82.62 53.41) (end 81.915 52.705) (width 0.3) (layer "F.Cu") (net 14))
 (segment (start 90.7825 53.41) (end 82.62 53.41) (width 0.3) (layer "F.Cu") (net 14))
 (segment (start 81.915 48.26) (end 83.185 46.99) (width 0.3) (layer "F.Cu") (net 14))
 (segment (start 84.455 48.26) (end 87.445 48.26) (width 0.3) (layer "F.Cu") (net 10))
 (segment (start 83.185 49.53) (end 84.455 48.26) (width 0.3) (layer "F.Cu") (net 10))
 (segment (start 87.445 45.72) (end 93.1725 51.4475) (width 0.3) (layer "F.Cu") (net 9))
 (segment (start 93.1725 51.4475) (end 93.1725 53.975) (width 0.3) (layer "F.Cu") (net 9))
 (segment (start 101.215 46.99) (end 99.945 45.72) (width 0.3) (layer "F.Cu") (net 3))
 (segment (start 101.215 46.99) (end 101.215 44.45) (width 0.3) (layer "F.Cu") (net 3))
 (segment (start 99.945 45.72) (end 96.52 45.72) (width 0.3) (layer "F.Cu") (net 3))
 (segment (start 109.22 50.5) (end 108.765 50.045) (width 0.3) (layer "F.Cu") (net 12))
 (segment (start 96.52 52.705) (end 96.52 50.8) (width 0.3) (layer "F.Cu") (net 12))
 (segment (start 109.22 52.07) (end 109.22 50.5) (width 0.3) (layer "F.Cu") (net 12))
 (via (at 96.52 52.705) (size 0.8) (drill 0.4) (layers "F.Cu" "B.Cu") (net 12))
 (via (at 109.22 52.07) (size 0.8) (drill 0.4) (layers "F.Cu" "B.Cu") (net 12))
 (segment (start 96.52 52.705) (end 108.585 52.705) (width 0.3) (layer "B.Cu") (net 12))
 (segment (start 108.585 52.705) (end 109.22 52.07) (width 0.3) (layer "B.Cu") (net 12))
 (segment (start 88.265 40.9975) (end 84.0975 40.9975) (width 0.3) (layer "F.Cu") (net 1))
 (segment (start 84.0975 40.9975) (end 83.185 41.91) (width 0.3) (layer "F.Cu") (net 1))
 (segment (start 95.25 36.195) (end 93.98 36.195) (width 0.3) (layer "F.Cu") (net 17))
 (segment (start 97.89 33.655) (end 97.79 33.655) (width 0.3) (layer "F.Cu") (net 17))
 (segment (start 97.79 33.655) (end 95.25 36.195) (width 0.3) (layer "F.Cu") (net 17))
 (segment (start 91.44 34.29) (end 92.075 33.655) (width 0.3) (layer "F.Cu") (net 18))
 (segment (start 92.075 33.655) (end 93.98 33.655) (width 0.3) (layer "F.Cu") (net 18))
 (segment (start 91.44 37.465) (end 91.44 34.29) (width 0.3) (layer "F.Cu") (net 18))
 (segment (start 97.89 36.195) (end 95.985 38.1) (width 0.3) (layer "F.Cu") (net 18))
 (segment (start 92.075 38.1) (end 91.44 37.465) (width 0.3) (layer "F.Cu") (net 18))
 (segment (start 95.985 38.1) (end 92.075 38.1) (width 0.3) (layer "F.Cu") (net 18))
 (segment (start 106.553 35.81) (end 104.425 35.81) (width 0.3) (layer "F.Cu") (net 7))
 (segment (start 104.425 35.81) (end 104.04 36.195) (width 0.3) (layer "F.Cu") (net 7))
 (segment (start 106.553 33.02) (end 104.675 33.02) (width 0.3) (layer "F.Cu") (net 5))
 (segment (start 104.675 33.02) (end 104.04 33.655) (width 0.3) (layer "F.Cu") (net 5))
 (segment (start 104.14 46.99) (end 104.14 50.8) (width 0.3) (layer "F.Cu") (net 4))
 (segment (start 112.17 43.815) (end 111.76 44.225) (width 0.3) (layer "F.Cu") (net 4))
 (segment (start 117.725 30.095) (end 111.125 30.095) (width 0.3) (layer "F.Cu") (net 4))
 (segment (start 104.14 44.45) (end 104.14 46.99) (width 0.3) (layer "F.Cu") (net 4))
 (segment (start 107.1898 44.225) (end 107.188 44.2232) (width 0.3) (layer "F.Cu") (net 4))
 (segment (start 111.76 44.225) (end 109.474 44.225) (width 0.3) (layer "F.Cu") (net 4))
 (segment (start 115.345 44.225) (end 111.76 44.225) (width 0.3) (layer "F.Cu") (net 4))
 (segment (start 119.38 48.26) (end 115.345 44.225) (width 0.3) (layer "F.Cu") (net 4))
 (segment (start 109.474 44.225) (end 107.1898 44.225) (width 0.3) (layer "F.Cu") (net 4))
 (segment (start 111.125 30.095) (end 106.553 30.095) (width 0.3) (layer "F.Cu") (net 4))
 (segment (start 119.38 31.75) (end 117.725 30.095) (width 0.3) (layer "F.Cu") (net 4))
 (segment (start 107.188 44.2232) (end 104.3668 44.2232) (width 0.3) (layer "F.Cu") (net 4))
 (segment (start 104.3668 44.2232) (end 104.14 44.45) (width 0.3) (layer "F.Cu") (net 4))
 (segment (start 119.38 36.83) (end 117.475 38.735) (width 0.3) (layer "F.Cu") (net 8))
 (segment (start 117.475 38.735) (end 106.553 38.735) (width 0.3) (layer "F.Cu") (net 8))
 (segment (start 80.645 39.37) (end 80.645 53.34) (width 0.3) (layer "F.Cu") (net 15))
 (segment (start 86.36 33.655) (end 80.645 39.37) (width 0.3) (layer "F.Cu") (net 15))
 (segment (start 81.915 54.61) (end 83.185 54.61) (width 0.3) (layer "F.Cu") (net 15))
 (segment (start 80.645 53.34) (end 81.915 54.61) (width 0.3) (layer "F.Cu") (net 15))
 (segment (start 83.185 52.07) (end 83.185 54.61) (width 0.3) (layer "B.Cu") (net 15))
 (segment (start 86.36 36.195) (end 90.17 40.005) (width 0.3) (layer "F.Cu") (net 2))
 (segment (start 90.17 42.545) (end 89.8925 42.8225) (width 0.3) (layer "F.Cu") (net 2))
 (segment (start 88.265 42.8225) (end 86.7175 42.8225) (width 0.3) (layer "F.Cu") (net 2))
 (segment (start 86.7175 42.8225) (end 85.09 44.45) (width 0.3) (layer "F.Cu") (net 2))
 (segment (start 89.8925 42.8225) (end 88.265 42.8225) (width 0.3) (layer "F.Cu") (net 2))
 (segment (start 85.09 44.45) (end 83.185 44.45) (width 0.3) (layer "F.Cu") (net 2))
 (segment (start 90.17 40.005) (end 90.17 42.545) (width 0.3) (layer "F.Cu") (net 2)))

